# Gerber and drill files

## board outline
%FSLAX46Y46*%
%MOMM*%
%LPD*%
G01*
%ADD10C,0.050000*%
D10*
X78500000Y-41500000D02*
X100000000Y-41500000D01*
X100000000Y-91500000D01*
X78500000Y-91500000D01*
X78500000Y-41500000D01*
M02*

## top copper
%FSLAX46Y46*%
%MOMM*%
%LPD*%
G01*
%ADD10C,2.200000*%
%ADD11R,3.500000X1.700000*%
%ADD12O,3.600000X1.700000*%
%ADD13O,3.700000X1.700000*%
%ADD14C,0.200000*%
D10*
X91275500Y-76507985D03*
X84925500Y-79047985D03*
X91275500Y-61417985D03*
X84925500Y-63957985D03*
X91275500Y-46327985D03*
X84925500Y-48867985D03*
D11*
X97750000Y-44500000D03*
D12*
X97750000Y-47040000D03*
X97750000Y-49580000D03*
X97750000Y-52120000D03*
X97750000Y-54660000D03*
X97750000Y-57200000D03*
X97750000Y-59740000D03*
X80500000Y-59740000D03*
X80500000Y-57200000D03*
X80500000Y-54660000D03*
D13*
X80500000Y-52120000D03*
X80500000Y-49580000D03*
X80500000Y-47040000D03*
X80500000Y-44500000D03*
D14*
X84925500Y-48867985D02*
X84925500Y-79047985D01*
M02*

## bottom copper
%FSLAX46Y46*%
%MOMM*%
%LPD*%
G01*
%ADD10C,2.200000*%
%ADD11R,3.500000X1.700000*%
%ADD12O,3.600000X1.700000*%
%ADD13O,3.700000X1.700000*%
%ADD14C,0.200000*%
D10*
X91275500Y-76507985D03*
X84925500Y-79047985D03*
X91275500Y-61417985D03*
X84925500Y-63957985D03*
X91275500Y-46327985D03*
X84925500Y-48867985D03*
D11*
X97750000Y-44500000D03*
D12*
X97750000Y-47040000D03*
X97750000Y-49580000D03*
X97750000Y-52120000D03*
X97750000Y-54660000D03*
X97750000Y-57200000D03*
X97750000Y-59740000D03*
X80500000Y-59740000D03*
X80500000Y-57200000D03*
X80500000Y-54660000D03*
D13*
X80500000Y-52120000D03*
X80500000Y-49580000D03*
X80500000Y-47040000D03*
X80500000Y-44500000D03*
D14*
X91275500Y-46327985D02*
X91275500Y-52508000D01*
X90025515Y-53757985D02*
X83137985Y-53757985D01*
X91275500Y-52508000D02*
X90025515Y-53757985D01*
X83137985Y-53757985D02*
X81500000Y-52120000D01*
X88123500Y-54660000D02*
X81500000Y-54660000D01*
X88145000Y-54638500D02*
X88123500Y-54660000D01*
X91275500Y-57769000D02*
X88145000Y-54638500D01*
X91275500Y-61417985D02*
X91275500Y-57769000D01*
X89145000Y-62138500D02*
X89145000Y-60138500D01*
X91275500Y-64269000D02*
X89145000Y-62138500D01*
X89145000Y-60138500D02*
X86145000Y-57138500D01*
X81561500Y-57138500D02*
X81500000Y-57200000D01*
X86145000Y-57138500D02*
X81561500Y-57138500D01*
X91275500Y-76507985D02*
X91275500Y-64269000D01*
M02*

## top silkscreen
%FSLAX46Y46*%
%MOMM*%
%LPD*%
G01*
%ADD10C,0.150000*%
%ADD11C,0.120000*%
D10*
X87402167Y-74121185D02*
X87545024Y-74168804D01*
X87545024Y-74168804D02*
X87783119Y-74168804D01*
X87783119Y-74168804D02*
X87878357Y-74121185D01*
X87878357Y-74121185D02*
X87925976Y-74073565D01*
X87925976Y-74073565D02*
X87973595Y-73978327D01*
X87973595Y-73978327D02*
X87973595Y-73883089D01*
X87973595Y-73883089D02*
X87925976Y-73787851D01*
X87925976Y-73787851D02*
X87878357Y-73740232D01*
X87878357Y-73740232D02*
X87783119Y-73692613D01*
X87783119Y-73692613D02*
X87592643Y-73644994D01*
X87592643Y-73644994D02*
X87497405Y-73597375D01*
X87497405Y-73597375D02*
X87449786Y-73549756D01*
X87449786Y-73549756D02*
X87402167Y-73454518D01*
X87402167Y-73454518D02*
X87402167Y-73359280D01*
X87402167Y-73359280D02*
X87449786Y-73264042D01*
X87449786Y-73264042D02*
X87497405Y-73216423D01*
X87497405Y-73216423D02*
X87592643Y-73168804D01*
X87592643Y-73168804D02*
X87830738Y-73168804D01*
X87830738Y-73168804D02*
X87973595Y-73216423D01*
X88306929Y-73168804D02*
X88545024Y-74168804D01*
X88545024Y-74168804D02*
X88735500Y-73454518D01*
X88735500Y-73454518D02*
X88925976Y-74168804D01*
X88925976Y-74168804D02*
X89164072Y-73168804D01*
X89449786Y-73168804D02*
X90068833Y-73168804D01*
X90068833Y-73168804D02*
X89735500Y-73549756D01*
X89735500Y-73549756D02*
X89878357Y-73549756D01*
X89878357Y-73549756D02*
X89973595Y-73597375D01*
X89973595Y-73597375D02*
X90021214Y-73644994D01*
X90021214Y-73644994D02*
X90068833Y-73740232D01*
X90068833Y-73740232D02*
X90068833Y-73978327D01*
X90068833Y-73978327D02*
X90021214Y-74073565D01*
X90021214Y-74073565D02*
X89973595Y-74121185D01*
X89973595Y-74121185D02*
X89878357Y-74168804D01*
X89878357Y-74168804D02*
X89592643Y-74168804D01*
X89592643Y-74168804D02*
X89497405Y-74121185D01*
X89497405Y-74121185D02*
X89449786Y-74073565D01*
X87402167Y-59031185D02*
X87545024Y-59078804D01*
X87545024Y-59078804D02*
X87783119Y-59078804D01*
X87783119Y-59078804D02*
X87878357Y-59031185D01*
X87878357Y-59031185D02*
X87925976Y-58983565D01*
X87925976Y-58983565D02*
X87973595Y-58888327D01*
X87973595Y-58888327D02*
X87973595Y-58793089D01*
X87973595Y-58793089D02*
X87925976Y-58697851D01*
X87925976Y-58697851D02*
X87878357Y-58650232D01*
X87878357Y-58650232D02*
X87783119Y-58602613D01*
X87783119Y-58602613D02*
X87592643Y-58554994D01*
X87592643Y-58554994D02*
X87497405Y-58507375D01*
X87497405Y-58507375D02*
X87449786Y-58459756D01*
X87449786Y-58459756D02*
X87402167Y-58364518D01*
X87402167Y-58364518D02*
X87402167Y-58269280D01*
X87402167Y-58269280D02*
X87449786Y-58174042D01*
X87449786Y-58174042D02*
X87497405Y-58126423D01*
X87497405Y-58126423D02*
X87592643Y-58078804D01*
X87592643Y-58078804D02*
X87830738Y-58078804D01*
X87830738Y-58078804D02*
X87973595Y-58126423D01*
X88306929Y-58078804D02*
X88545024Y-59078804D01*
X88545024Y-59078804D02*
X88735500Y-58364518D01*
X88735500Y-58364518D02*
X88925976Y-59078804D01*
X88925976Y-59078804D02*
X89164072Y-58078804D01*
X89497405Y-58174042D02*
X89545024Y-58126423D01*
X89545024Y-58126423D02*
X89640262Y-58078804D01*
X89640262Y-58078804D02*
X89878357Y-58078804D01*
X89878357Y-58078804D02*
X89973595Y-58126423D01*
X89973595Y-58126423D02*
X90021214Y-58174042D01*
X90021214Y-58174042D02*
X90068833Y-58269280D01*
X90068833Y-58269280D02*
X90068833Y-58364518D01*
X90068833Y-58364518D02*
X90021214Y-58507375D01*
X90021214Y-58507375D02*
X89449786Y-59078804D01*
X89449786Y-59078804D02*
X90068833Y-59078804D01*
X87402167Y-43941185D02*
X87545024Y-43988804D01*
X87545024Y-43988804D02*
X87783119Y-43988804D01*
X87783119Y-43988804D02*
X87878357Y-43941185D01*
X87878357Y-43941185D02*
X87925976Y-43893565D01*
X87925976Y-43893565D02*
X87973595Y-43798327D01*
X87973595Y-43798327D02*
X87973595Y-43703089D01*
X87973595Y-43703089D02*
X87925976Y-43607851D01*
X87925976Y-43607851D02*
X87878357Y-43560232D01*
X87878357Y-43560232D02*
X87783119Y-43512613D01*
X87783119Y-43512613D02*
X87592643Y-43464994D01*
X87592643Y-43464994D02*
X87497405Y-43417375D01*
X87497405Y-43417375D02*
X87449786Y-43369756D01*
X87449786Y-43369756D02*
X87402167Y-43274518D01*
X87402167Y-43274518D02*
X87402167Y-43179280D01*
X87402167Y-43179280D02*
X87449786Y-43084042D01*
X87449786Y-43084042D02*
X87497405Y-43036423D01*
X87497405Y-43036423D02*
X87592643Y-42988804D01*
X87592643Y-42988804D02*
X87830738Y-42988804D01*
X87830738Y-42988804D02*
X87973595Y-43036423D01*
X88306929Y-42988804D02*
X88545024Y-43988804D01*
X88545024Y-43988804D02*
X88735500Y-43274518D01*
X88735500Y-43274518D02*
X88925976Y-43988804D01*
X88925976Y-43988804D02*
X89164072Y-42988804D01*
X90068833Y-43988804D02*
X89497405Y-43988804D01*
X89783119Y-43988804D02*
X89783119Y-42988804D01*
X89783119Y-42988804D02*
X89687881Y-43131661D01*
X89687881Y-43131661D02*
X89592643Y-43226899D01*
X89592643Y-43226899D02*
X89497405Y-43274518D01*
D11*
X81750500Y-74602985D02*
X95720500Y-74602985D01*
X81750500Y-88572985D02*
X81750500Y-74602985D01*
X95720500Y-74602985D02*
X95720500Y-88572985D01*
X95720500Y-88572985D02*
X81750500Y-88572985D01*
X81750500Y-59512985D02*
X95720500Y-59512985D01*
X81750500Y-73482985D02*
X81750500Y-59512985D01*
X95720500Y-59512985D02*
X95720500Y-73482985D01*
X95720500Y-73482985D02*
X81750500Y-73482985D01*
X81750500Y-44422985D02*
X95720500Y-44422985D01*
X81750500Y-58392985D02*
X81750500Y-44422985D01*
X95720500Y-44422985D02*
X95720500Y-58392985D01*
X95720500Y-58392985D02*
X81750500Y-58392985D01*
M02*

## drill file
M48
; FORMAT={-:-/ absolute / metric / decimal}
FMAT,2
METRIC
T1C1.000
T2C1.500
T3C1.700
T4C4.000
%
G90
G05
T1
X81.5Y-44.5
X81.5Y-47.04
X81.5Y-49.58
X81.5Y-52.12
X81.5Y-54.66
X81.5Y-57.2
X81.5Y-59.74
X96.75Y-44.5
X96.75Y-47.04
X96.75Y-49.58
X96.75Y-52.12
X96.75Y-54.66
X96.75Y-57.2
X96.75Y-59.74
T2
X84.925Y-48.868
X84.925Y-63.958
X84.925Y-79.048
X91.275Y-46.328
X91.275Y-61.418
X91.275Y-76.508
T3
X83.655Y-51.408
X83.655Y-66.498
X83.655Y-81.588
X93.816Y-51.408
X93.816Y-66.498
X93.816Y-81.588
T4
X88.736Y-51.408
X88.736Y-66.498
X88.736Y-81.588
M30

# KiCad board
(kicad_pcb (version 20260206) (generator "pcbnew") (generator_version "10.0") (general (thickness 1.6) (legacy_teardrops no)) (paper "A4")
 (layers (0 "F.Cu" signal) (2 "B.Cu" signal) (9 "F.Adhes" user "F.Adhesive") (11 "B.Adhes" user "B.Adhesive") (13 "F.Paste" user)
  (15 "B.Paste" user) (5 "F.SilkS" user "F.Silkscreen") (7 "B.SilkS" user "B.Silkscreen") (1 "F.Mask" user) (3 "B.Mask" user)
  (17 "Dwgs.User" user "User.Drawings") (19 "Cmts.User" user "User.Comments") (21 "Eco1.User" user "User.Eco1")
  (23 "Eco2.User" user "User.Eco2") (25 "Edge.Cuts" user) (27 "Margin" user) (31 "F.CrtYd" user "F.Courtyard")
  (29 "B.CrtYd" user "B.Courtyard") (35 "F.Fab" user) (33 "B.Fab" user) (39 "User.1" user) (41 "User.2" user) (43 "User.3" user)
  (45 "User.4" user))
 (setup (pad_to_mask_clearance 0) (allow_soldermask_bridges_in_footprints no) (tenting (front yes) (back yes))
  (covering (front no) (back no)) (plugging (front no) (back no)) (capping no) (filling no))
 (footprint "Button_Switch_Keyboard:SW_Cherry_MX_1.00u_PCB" (layer "F.Cu") (at 91.2755 76.507985)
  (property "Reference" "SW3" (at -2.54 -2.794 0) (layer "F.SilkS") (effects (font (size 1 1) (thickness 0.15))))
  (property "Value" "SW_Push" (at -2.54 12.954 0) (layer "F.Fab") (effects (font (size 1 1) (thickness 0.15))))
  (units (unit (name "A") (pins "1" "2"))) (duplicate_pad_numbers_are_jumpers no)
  (fp_line (start -9.525 -1.905) (end 4.445 -1.905) (stroke (width 0.12) (type solid)) (layer "F.SilkS"))
  (fp_line (start -9.525 12.065) (end -9.525 -1.905) (stroke (width 0.12) (type solid)) (layer "F.SilkS"))
  (fp_line (start 4.445 -1.905) (end 4.445 12.065) (stroke (width 0.12) (type solid)) (layer "F.SilkS"))
  (fp_line (start 4.445 12.065) (end -9.525 12.065) (stroke (width 0.12) (type solid)) (layer "F.SilkS"))
  (pad "" np_thru_hole circle (at -7.62 5.08) (size 1.7 1.7) (drill 1.7) (layers "*.Cu" "*.Mask"))
  (pad "" np_thru_hole circle (at -2.54 5.08) (size 4 4) (drill 4) (layers "*.Cu" "*.Mask"))
  (pad "" np_thru_hole circle (at 2.54 5.08) (size 1.7 1.7) (drill 1.7) (layers "*.Cu" "*.Mask"))
  (pad "1" thru_hole circle (at 0 0) (size 2.2 2.2) (drill 1.5) (layers "*.Cu" "*.Mask") (remove_unused_layers no)
   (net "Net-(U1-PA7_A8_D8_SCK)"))
  (pad "2" thru_hole circle (at -6.35 2.54) (size 2.2 2.2) (drill 1.5) (layers "*.Cu" "*.Mask") (remove_unused_layers no) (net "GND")))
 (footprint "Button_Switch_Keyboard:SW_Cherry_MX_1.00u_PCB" (layer "F.Cu") (at 91.2755 61.417985)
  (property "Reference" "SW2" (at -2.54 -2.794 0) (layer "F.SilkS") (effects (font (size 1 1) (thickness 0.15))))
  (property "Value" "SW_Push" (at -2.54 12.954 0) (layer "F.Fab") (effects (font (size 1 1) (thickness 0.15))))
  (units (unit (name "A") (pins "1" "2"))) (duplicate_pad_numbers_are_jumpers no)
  (fp_line (start -9.525 -1.905) (end 4.445 -1.905) (stroke (width 0.12) (type solid)) (layer "F.SilkS"))
  (fp_line (start -9.525 12.065) (end -9.525 -1.905) (stroke (width 0.12) (type solid)) (layer "F.SilkS"))
  (fp_line (start 4.445 -1.905) (end 4.445 12.065) (stroke (width 0.12) (type solid)) (layer "F.SilkS"))
  (fp_line (start 4.445 12.065) (end -9.525 12.065) (stroke (width 0.12) (type solid)) (layer "F.SilkS"))
  (pad "" np_thru_hole circle (at -7.62 5.08) (size 1.7 1.7) (drill 1.7) (layers "*.Cu" "*.Mask"))
  (pad "" np_thru_hole circle (at -2.54 5.08) (size 4 4) (drill 4) (layers "*.Cu" "*.Mask"))
  (pad "" np_thru_hole circle (at 2.54 5.08) (size 1.7 1.7) (drill 1.7) (layers "*.Cu" "*.Mask"))
  (pad "1" thru_hole circle (at 0 0) (size 2.2 2.2) (drill 1.5) (layers "*.Cu" "*.Mask") (remove_unused_layers no)
   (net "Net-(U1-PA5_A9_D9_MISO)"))
  (pad "2" thru_hole circle (at -6.35 2.54) (size 2.2 2.2) (drill 1.5) (layers "*.Cu" "*.Mask") (remove_unused_layers no) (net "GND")))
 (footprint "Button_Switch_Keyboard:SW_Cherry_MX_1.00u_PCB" (layer "F.Cu") (at 91.2755 46.327985)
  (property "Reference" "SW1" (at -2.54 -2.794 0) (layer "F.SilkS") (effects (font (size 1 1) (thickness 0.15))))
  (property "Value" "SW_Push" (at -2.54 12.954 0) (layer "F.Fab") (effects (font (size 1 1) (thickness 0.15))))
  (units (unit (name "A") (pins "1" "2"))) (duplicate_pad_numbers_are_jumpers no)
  (fp_line (start -9.525 -1.905) (end 4.445 -1.905) (stroke (width 0.12) (type solid)) (layer "F.SilkS"))
  (fp_line (start -9.525 12.065) (end -9.525 -1.905) (stroke (width 0.12) (type solid)) (layer "F.SilkS"))
  (fp_line (start 4.445 -1.905) (end 4.445 12.065) (stroke (width 0.12) (type solid)) (layer "F.SilkS"))
  (fp_line (start 4.445 12.065) (end -9.525 12.065) (stroke (width 0.12) (type solid)) (layer "F.SilkS"))
  (pad "" np_thru_hole circle (at -7.62 5.08) (size 1.7 1.7) (drill 1.7) (layers "*.Cu" "*.Mask"))
  (pad "" np_thru_hole circle (at -2.54 5.08) (size 4 4) (drill 4) (layers "*.Cu" "*.Mask"))
  (pad "" np_thru_hole circle (at 2.54 5.08) (size 1.7 1.7) (drill 1.7) (layers "*.Cu" "*.Mask"))
  (pad "1" thru_hole circle (at 0 0) (size 2.2 2.2) (drill 1.5) (layers "*.Cu" "*.Mask") (remove_unused_layers no)
   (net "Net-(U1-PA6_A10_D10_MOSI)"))
  (pad "2" thru_hole circle (at -6.35 2.54) (size 2.2 2.2) (drill 1.5) (layers "*.Cu" "*.Mask") (remove_unused_layers no) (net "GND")))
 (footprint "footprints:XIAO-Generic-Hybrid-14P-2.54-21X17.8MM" (layer "B.Cu") (at 89.125 52.12 180)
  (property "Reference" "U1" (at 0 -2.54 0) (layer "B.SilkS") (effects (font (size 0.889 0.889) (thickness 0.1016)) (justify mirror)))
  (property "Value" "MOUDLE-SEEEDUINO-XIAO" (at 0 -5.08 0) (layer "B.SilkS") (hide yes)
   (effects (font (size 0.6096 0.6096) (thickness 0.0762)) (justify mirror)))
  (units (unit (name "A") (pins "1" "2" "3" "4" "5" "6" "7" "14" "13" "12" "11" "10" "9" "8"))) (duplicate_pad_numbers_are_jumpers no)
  (pad "1" thru_hole rect (at -7.625 7.62 180) (size 3.5 1.7) (drill 1 (offset -1 0)) (layers "*.Cu" "*.Mask") (remove_unused_layers no)
   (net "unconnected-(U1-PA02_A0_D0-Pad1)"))
  (pad "2" thru_hole oval (at -7.625 5.08 180) (size 3.6 1.7) (drill 1 (offset -1 0)) (layers "*.Cu" "*.Mask") (remove_unused_layers no)
   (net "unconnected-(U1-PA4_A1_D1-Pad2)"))
  (pad "3" thru_hole oval (at -7.625 2.54 180) (size 3.6 1.7) (drill 1 (offset -1 0)) (layers "*.Cu" "*.Mask") (remove_unused_layers no)
   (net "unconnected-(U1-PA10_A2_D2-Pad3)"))
  (pad "4" thru_hole oval (at -7.625 0 180) (size 3.6 1.7) (drill 1 (offset -1 0)) (layers "*.Cu" "*.Mask") (remove_unused_layers no)
   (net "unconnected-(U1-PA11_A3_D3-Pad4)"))
  (pad "5" thru_hole oval (at -7.625 -2.54 180) (size 3.6 1.7) (drill 1 (offset -1 0)) (layers "*.Cu" "*.Mask") (remove_unused_layers no)
   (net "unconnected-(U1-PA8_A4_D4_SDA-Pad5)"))
  (pad "6" thru_hole oval (at -7.625 -5.08) (size 3.6 1.7) (drill 1 (offset 1 0)) (layers "*.Cu" "*.Mask") (remove_unused_layers no)
   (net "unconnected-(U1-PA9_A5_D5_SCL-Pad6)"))
  (pad "7" thru_hole oval (at -7.625 -7.62 180) (size 3.6 1.7) (drill 1 (offset -1 0)) (layers "*.Cu" "*.Mask") (remove_unused_layers no)
   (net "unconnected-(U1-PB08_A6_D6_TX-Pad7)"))
  (pad "8" thru_hole oval (at 7.625 -7.62 180) (size 3.6 1.7) (drill 1 (offset 1 0)) (layers "*.Cu" "*.Mask") (remove_unused_layers no)
   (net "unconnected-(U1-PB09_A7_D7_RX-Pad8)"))
  (pad "9" thru_hole oval (at 7.625 -5.08 180) (size 3.6 1.7) (drill 1 (offset 1 0)) (layers "*.Cu" "*.Mask") (remove_unused_layers no)
   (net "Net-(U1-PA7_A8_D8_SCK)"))
  (pad "10" thru_hole oval (at 7.625 -2.54 180) (size 3.6 1.7) (drill 1 (offset 1 0)) (layers "*.Cu" "*.Mask") (remove_unused_layers no)
   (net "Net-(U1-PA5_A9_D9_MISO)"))
  (pad "11" thru_hole oval (at 7.625 0 180) (size 3.7 1.7) (drill 1 (offset 1 0)) (layers "*.Cu" "*.Mask") (remove_unused_layers no)
   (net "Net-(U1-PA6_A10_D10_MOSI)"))
  (pad "12" thru_hole oval (at 7.625 2.54 180) (size 3.7 1.7) (drill 1 (offset 1 0)) (layers "*.Cu" "*.Mask") (remove_unused_layers no)
   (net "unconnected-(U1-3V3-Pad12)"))
  (pad "13" thru_hole oval (at 7.625 5.08 180) (size 3.7 1.7) (drill 1 (offset 1 0)) (layers "*.Cu" "*.Mask") (remove_unused_layers no)
   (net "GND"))
  (pad "14" thru_hole oval (at 7.625 7.62 180) (size 3.7 1.7) (drill 1 (offset 1 0)) (layers "*.Cu" "*.Mask") (remove_unused_layers no)
   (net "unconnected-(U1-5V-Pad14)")))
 (gr_rect (start 78.5 41.5) (end 100 91.5) (stroke (width 0.05) (type default)) (fill no) (layer "Edge.Cuts"))
 (segment (start 91.2755 46.327985) (end 91.2755 52.508) (width 0.2) (layer "B.Cu") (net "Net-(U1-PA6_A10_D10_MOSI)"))
 (segment (start 90.025515 53.757985) (end 83.137985 53.757985) (width 0.2) (layer "B.Cu") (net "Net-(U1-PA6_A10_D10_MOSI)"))
 (segment (start 91.2755 52.508) (end 90.025515 53.757985) (width 0.2) (layer "B.Cu") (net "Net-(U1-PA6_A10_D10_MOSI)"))
 (segment (start 83.137985 53.757985) (end 81.5 52.12) (width 0.2) (layer "B.Cu") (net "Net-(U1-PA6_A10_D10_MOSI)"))
 (segment (start 84.9255 48.867985) (end 84.9255 79.047985) (width 0.2) (layer "F.Cu") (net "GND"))
 (segment (start 88.1235 54.66) (end 81.5 54.66) (width 0.2) (layer "B.Cu") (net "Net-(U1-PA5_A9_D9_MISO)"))
 (segment (start 88.145 54.6385) (end 88.1235 54.66) (width 0.2) (layer "B.Cu") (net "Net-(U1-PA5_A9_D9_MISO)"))
 (segment (start 91.2755 57.769) (end 88.145 54.6385) (width 0.2) (layer "B.Cu") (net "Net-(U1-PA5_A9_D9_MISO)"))
 (segment (start 91.2755 61.417985) (end 91.2755 57.769) (width 0.2) (layer "B.Cu") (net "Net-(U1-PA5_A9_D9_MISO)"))
 (segment (start 89.145 62.1385) (end 89.145 60.1385) (width 0.2) (layer "B.Cu") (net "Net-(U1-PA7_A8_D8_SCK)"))
 (segment (start 91.2755 64.269) (end 89.145 62.1385) (width 0.2) (layer "B.Cu") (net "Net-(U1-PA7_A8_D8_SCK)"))
 (segment (start 89.145 60.1385) (end 86.145 57.1385) (width 0.2) (layer "B.Cu") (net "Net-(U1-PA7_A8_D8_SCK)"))
 (segment (start 81.5615 57.1385) (end 81.5 57.2) (width 0.2) (layer "B.Cu") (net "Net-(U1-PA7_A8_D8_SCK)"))
 (segment (start 86.145 57.1385) (end 81.5615 57.1385) (width 0.2) (layer "B.Cu") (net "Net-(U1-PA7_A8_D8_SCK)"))
 (segment (start 91.2755 76.507985) (end 91.2755 64.269) (width 0.2) (layer "B.Cu") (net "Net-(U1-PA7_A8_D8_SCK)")))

